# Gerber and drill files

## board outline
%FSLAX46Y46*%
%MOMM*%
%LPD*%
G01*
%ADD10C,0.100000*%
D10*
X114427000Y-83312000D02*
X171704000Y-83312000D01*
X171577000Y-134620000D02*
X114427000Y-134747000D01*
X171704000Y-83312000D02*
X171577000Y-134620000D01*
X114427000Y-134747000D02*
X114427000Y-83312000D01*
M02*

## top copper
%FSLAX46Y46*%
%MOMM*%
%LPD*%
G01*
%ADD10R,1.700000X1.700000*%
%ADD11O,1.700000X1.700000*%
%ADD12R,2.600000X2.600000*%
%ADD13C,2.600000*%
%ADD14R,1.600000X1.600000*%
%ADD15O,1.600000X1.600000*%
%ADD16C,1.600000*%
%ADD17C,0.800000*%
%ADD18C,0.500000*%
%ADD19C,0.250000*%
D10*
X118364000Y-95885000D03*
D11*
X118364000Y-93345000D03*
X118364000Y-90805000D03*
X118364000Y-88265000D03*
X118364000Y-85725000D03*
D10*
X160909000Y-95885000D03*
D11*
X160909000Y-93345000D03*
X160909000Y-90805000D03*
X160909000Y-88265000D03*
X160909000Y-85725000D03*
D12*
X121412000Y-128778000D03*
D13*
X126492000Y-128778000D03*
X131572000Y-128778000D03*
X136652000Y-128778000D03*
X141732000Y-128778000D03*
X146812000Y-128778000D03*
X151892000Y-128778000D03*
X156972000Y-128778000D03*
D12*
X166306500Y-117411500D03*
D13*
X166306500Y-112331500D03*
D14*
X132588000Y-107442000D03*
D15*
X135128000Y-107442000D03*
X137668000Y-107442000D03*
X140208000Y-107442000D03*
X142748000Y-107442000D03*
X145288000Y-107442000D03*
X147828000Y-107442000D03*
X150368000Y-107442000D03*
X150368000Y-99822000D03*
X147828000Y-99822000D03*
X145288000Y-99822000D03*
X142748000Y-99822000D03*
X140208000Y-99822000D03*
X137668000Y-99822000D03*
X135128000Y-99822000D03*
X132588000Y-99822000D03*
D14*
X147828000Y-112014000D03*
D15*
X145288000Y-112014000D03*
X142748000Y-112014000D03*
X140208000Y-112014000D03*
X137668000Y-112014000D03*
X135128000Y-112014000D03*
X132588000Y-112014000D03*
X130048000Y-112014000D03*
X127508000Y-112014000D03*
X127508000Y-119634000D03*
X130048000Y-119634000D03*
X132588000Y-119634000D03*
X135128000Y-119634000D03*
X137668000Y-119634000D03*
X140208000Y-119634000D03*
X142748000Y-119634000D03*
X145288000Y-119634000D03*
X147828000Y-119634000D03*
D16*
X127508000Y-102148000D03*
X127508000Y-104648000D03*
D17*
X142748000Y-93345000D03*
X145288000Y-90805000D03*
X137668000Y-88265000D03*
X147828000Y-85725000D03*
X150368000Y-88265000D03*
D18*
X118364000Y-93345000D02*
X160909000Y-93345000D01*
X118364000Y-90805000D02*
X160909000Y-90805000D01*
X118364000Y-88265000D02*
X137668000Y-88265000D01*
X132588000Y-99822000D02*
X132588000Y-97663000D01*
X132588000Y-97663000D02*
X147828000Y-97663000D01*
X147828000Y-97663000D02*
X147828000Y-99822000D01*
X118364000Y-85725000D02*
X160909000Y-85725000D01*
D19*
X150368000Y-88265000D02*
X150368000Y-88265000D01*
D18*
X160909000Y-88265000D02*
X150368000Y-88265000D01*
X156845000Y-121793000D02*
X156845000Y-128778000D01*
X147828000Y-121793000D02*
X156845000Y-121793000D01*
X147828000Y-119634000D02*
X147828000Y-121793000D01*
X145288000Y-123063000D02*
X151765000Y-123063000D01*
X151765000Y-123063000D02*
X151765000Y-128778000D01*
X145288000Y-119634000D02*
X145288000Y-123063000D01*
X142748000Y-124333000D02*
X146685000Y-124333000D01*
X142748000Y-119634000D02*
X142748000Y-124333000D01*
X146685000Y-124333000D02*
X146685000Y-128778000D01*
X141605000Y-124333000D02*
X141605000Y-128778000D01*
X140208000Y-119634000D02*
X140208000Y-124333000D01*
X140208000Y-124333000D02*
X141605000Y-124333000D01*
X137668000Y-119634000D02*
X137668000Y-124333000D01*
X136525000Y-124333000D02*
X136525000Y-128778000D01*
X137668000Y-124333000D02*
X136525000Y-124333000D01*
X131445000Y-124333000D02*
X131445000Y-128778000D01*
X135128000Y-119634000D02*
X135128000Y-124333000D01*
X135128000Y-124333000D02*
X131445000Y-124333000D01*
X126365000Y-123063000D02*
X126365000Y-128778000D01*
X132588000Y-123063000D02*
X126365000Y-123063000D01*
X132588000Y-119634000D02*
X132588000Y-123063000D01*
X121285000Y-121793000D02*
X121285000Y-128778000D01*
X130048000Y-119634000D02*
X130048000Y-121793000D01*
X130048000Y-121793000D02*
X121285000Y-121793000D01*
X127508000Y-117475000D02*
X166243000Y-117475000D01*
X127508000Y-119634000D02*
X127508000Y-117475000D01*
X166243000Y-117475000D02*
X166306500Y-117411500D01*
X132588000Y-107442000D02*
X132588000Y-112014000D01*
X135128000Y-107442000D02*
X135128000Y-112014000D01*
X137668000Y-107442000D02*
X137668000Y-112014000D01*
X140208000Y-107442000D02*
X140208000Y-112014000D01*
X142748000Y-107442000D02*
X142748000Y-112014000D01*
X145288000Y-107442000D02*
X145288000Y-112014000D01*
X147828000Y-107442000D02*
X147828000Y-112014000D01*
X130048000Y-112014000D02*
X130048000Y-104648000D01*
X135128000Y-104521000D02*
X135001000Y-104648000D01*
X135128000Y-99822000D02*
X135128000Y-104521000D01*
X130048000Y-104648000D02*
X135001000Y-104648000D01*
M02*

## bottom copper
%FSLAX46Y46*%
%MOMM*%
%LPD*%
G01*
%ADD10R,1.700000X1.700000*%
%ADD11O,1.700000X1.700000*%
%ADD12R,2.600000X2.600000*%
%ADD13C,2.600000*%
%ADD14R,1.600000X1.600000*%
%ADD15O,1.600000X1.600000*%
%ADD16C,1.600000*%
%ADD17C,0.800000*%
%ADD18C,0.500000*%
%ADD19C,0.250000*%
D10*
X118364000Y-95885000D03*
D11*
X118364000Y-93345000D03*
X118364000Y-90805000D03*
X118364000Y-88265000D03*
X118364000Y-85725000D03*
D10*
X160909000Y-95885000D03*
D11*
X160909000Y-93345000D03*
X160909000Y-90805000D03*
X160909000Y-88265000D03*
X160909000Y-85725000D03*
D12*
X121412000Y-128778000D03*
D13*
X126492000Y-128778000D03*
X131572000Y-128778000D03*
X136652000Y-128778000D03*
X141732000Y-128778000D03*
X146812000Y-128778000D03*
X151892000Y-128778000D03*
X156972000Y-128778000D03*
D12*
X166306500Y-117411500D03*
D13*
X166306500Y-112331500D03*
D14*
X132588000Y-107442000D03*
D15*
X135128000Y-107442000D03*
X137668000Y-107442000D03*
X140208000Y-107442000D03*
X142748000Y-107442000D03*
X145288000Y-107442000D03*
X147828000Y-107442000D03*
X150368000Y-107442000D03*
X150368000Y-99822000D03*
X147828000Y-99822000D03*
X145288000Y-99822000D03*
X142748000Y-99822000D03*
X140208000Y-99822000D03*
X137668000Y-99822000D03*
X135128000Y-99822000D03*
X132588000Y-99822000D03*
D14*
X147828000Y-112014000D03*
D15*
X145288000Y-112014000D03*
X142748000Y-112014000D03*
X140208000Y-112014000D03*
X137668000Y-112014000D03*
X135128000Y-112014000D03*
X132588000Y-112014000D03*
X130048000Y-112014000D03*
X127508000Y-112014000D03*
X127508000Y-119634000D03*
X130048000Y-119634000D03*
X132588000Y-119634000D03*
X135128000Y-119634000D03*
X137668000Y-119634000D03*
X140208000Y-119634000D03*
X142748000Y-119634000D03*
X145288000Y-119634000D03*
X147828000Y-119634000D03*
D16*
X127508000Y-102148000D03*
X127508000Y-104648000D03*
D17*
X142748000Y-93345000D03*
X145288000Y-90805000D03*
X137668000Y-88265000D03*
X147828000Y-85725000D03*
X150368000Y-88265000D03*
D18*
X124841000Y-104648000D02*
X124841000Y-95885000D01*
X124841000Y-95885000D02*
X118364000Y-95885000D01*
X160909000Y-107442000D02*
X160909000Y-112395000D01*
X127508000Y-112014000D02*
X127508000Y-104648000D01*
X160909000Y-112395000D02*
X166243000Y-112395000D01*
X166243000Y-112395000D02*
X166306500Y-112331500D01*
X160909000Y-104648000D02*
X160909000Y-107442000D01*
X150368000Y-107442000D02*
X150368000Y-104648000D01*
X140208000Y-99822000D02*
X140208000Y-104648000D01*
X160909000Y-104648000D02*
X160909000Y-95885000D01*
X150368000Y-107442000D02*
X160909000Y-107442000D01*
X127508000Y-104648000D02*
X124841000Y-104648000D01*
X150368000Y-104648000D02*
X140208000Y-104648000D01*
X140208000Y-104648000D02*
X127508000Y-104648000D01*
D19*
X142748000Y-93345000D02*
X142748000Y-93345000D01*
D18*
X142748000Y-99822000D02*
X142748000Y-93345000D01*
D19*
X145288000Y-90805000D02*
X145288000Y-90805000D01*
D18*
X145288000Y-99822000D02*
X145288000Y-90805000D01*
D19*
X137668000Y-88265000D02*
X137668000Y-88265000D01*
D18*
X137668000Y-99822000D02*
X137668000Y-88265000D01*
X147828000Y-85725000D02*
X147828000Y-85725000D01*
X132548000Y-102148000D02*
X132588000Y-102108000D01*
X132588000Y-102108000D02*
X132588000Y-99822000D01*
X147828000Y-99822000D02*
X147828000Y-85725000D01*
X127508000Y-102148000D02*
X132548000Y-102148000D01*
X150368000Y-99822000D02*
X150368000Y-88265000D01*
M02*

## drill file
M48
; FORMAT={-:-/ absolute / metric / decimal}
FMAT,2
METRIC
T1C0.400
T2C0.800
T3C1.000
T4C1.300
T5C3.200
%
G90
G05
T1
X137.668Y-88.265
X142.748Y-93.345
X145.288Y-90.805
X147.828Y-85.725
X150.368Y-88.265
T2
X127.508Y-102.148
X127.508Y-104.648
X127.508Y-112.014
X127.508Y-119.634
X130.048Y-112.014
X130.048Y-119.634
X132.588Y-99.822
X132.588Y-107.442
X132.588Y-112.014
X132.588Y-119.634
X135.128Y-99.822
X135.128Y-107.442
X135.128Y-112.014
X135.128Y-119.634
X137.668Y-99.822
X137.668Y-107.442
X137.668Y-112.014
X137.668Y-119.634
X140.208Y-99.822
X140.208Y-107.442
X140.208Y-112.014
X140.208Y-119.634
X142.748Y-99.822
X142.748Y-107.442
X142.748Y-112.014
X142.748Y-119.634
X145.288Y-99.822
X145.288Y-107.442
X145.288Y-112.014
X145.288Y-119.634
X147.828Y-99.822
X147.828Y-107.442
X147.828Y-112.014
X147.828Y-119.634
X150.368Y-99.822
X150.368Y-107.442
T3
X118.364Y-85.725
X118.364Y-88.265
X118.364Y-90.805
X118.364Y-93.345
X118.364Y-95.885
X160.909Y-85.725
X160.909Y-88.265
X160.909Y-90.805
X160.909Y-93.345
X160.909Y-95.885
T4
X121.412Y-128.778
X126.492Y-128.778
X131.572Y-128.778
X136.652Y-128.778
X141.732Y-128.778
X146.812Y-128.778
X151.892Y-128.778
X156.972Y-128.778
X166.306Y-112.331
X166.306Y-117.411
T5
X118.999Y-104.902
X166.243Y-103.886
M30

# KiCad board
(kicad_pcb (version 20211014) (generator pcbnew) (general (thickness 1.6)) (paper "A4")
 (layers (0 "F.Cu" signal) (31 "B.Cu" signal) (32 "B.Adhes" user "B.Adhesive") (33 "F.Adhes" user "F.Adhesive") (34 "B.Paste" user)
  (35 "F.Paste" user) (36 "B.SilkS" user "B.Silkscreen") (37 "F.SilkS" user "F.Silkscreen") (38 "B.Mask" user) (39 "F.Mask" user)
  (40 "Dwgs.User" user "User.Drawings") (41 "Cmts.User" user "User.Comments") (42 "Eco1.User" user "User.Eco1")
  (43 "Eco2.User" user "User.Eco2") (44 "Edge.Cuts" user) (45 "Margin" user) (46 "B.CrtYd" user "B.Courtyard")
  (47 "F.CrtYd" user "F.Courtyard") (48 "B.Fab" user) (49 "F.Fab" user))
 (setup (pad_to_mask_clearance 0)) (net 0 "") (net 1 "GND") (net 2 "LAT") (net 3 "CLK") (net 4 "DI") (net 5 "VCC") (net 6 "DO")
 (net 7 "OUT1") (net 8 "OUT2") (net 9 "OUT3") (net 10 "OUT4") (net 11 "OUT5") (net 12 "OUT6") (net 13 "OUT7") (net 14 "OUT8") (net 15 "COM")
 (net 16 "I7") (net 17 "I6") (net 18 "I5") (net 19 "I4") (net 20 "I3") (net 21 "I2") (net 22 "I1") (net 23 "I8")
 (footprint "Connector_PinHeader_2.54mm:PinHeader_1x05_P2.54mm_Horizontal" (layer "F.Cu") (at 118.364 95.885 180)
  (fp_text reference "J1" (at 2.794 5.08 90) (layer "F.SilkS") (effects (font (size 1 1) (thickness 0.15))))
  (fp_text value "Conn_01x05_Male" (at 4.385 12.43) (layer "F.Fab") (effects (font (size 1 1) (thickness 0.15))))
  (pad "1" thru_hole rect locked (at 0 0 180) (size 1.7 1.7) (drill 1) (layers *.Cu *.Mask) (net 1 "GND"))
  (pad "2" thru_hole oval locked (at 0 2.54 180) (size 1.7 1.7) (drill 1) (layers *.Cu *.Mask) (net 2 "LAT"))
  (pad "3" thru_hole oval locked (at 0 5.08 180) (size 1.7 1.7) (drill 1) (layers *.Cu *.Mask) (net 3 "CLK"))
  (pad "4" thru_hole oval locked (at 0 7.62 180) (size 1.7 1.7) (drill 1) (layers *.Cu *.Mask) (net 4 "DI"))
  (pad "5" thru_hole oval locked (at 0 10.16 180) (size 1.7 1.7) (drill 1) (layers *.Cu *.Mask) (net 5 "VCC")))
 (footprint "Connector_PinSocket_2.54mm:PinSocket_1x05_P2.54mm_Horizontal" (layer "F.Cu") (at 160.909 95.885 180)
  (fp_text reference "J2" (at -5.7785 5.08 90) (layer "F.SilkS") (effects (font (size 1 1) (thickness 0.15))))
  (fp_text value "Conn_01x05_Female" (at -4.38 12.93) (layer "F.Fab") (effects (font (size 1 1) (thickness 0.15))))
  (pad "1" thru_hole rect locked (at 0 0 180) (size 1.7 1.7) (drill 1) (layers *.Cu *.Mask) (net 1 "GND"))
  (pad "2" thru_hole oval locked (at 0 2.54 180) (size 1.7 1.7) (drill 1) (layers *.Cu *.Mask) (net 2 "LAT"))
  (pad "3" thru_hole oval locked (at 0 5.08 180) (size 1.7 1.7) (drill 1) (layers *.Cu *.Mask) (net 3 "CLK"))
  (pad "4" thru_hole oval locked (at 0 7.62 180) (size 1.7 1.7) (drill 1) (layers *.Cu *.Mask) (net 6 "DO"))
  (pad "5" thru_hole oval locked (at 0 10.16 180) (size 1.7 1.7) (drill 1) (layers *.Cu *.Mask) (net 5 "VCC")))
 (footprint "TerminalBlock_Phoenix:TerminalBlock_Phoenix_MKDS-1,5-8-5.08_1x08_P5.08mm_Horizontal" (layer "F.Cu") (at 121.412 128.778)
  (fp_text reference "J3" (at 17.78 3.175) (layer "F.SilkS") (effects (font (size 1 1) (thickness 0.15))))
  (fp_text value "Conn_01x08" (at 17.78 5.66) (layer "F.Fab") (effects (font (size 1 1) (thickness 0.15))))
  (pad "1" thru_hole rect locked (at 0 0) (size 2.6 2.6) (drill 1.3) (layers *.Cu *.Mask) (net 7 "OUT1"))
  (pad "2" thru_hole circle locked (at 5.08 0) (size 2.6 2.6) (drill 1.3) (layers *.Cu *.Mask) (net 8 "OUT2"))
  (pad "3" thru_hole circle locked (at 10.16 0) (size 2.6 2.6) (drill 1.3) (layers *.Cu *.Mask) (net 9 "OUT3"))
  (pad "4" thru_hole circle locked (at 15.24 0) (size 2.6 2.6) (drill 1.3) (layers *.Cu *.Mask) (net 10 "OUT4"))
  (pad "5" thru_hole circle locked (at 20.32 0) (size 2.6 2.6) (drill 1.3) (layers *.Cu *.Mask) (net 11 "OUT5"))
  (pad "6" thru_hole circle locked (at 25.4 0) (size 2.6 2.6) (drill 1.3) (layers *.Cu *.Mask) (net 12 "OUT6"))
  (pad "7" thru_hole circle locked (at 30.48 0) (size 2.6 2.6) (drill 1.3) (layers *.Cu *.Mask) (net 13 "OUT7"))
  (pad "8" thru_hole circle locked (at 35.56 0) (size 2.6 2.6) (drill 1.3) (layers *.Cu *.Mask) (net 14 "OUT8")))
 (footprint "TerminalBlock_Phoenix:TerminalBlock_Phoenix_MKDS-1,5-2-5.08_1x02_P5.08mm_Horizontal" (layer "F.Cu") (at 166.3065 117.4115 90)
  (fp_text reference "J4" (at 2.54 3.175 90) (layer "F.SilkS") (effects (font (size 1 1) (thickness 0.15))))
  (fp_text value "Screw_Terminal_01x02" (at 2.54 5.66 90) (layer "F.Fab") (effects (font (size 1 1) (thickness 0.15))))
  (pad "1" thru_hole rect locked (at 0 0 90) (size 2.6 2.6) (drill 1.3) (layers *.Cu *.Mask) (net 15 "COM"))
  (pad "2" thru_hole circle locked (at 5.08 0 90) (size 2.6 2.6) (drill 1.3) (layers *.Cu *.Mask) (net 1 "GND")))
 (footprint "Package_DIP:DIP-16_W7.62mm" (layer "F.Cu") (at 132.588 107.442 90)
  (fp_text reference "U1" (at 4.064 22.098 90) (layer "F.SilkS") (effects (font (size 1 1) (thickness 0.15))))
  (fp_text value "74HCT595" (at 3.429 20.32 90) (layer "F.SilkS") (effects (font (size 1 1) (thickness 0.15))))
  (pad "1" thru_hole rect locked (at 0 0 90) (size 1.6 1.6) (drill 0.8) (layers *.Cu *.Mask) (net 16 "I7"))
  (pad "2" thru_hole oval locked (at 0 2.54 90) (size 1.6 1.6) (drill 0.8) (layers *.Cu *.Mask) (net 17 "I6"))
  (pad "3" thru_hole oval locked (at 0 5.08 90) (size 1.6 1.6) (drill 0.8) (layers *.Cu *.Mask) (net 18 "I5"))
  (pad "4" thru_hole oval locked (at 0 7.62 90) (size 1.6 1.6) (drill 0.8) (layers *.Cu *.Mask) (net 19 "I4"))
  (pad "5" thru_hole oval locked (at 0 10.16 90) (size 1.6 1.6) (drill 0.8) (layers *.Cu *.Mask) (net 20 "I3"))
  (pad "6" thru_hole oval locked (at 0 12.7 90) (size 1.6 1.6) (drill 0.8) (layers *.Cu *.Mask) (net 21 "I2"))
  (pad "7" thru_hole oval locked (at 0 15.24 90) (size 1.6 1.6) (drill 0.8) (layers *.Cu *.Mask) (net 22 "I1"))
  (pad "8" thru_hole oval locked (at 0 17.78 90) (size 1.6 1.6) (drill 0.8) (layers *.Cu *.Mask) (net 1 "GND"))
  (pad "9" thru_hole oval locked (at 7.62 17.78 90) (size 1.6 1.6) (drill 0.8) (layers *.Cu *.Mask) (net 6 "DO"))
  (pad "10" thru_hole oval locked (at 7.62 15.24 90) (size 1.6 1.6) (drill 0.8) (layers *.Cu *.Mask) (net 5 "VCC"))
  (pad "11" thru_hole oval locked (at 7.62 12.7 90) (size 1.6 1.6) (drill 0.8) (layers *.Cu *.Mask) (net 3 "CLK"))
  (pad "12" thru_hole oval locked (at 7.62 10.16 90) (size 1.6 1.6) (drill 0.8) (layers *.Cu *.Mask) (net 2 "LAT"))
  (pad "13" thru_hole oval locked (at 7.62 7.62 90) (size 1.6 1.6) (drill 0.8) (layers *.Cu *.Mask) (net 1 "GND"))
  (pad "14" thru_hole oval locked (at 7.62 5.08 90) (size 1.6 1.6) (drill 0.8) (layers *.Cu *.Mask) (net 4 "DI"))
  (pad "15" thru_hole oval locked (at 7.62 2.54 90) (size 1.6 1.6) (drill 0.8) (layers *.Cu *.Mask) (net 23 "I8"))
  (pad "16" thru_hole oval locked (at 7.62 0 90) (size 1.6 1.6) (drill 0.8) (layers *.Cu *.Mask) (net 5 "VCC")))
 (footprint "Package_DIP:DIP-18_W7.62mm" (layer "F.Cu") (at 147.828 112.014 -90)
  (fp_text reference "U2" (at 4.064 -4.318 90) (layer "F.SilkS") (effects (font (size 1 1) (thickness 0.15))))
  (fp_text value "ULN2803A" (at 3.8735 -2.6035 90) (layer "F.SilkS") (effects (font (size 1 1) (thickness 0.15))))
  (pad "1" thru_hole rect locked (at 0 0 270) (size 1.6 1.6) (drill 0.8) (layers *.Cu *.Mask) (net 22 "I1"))
  (pad "2" thru_hole oval locked (at 0 2.54 270) (size 1.6 1.6) (drill 0.8) (layers *.Cu *.Mask) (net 21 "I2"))
  (pad "3" thru_hole oval locked (at 0 5.08 270) (size 1.6 1.6) (drill 0.8) (layers *.Cu *.Mask) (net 20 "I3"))
  (pad "4" thru_hole oval locked (at 0 7.62 270) (size 1.6 1.6) (drill 0.8) (layers *.Cu *.Mask) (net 19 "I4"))
  (pad "5" thru_hole oval locked (at 0 10.16 270) (size 1.6 1.6) (drill 0.8) (layers *.Cu *.Mask) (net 18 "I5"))
  (pad "6" thru_hole oval locked (at 0 12.7 270) (size 1.6 1.6) (drill 0.8) (layers *.Cu *.Mask) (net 17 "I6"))
  (pad "7" thru_hole oval locked (at 0 15.24 270) (size 1.6 1.6) (drill 0.8) (layers *.Cu *.Mask) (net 16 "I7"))
  (pad "8" thru_hole oval locked (at 0 17.78 270) (size 1.6 1.6) (drill 0.8) (layers *.Cu *.Mask) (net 23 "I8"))
  (pad "9" thru_hole oval locked (at 0 20.32 270) (size 1.6 1.6) (drill 0.8) (layers *.Cu *.Mask) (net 1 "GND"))
  (pad "10" thru_hole oval locked (at 7.62 20.32 270) (size 1.6 1.6) (drill 0.8) (layers *.Cu *.Mask) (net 15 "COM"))
  (pad "11" thru_hole oval locked (at 7.62 17.78 270) (size 1.6 1.6) (drill 0.8) (layers *.Cu *.Mask) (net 7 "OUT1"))
  (pad "12" thru_hole oval locked (at 7.62 15.24 270) (size 1.6 1.6) (drill 0.8) (layers *.Cu *.Mask) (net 8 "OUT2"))
  (pad "13" thru_hole oval locked (at 7.62 12.7 270) (size 1.6 1.6) (drill 0.8) (layers *.Cu *.Mask) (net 9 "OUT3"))
  (pad "14" thru_hole oval locked (at 7.62 10.16 270) (size 1.6 1.6) (drill 0.8) (layers *.Cu *.Mask) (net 10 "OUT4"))
  (pad "15" thru_hole oval locked (at 7.62 7.62 270) (size 1.6 1.6) (drill 0.8) (layers *.Cu *.Mask) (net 11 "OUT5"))
  (pad "16" thru_hole oval locked (at 7.62 5.08 270) (size 1.6 1.6) (drill 0.8) (layers *.Cu *.Mask) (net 12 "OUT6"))
  (pad "17" thru_hole oval locked (at 7.62 2.54 270) (size 1.6 1.6) (drill 0.8) (layers *.Cu *.Mask) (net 13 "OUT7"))
  (pad "18" thru_hole oval locked (at 7.62 0 270) (size 1.6 1.6) (drill 0.8) (layers *.Cu *.Mask) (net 14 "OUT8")))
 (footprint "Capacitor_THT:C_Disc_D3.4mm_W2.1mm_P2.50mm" (layer "F.Cu") (at 127.508 102.148 -90)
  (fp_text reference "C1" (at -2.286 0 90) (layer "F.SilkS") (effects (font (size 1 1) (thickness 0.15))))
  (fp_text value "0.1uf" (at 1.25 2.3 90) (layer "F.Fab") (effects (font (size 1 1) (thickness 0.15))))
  (pad "1" thru_hole circle locked (at 0 0 270) (size 1.6 1.6) (drill 0.8) (layers *.Cu *.Mask) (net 5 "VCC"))
  (pad "2" thru_hole circle locked (at 2.5 0 270) (size 1.6 1.6) (drill 0.8) (layers *.Cu *.Mask) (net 1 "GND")))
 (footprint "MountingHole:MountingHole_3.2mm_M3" (layer "F.Cu") (at 118.999 104.902)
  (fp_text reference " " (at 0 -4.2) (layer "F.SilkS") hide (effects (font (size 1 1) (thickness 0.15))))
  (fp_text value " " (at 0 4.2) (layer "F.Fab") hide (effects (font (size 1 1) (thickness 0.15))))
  (pad "" np_thru_hole circle locked (at 0 0) (size 3.2 3.2) (drill 3.2) (layers *.Cu *.Mask)))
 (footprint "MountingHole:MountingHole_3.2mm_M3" (layer "F.Cu") (at 166.243 103.886)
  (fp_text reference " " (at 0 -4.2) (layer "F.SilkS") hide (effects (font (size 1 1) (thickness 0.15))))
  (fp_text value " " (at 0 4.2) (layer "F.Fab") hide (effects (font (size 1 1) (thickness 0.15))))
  (pad "" np_thru_hole circle locked (at 0 0) (size 3.2 3.2) (drill 3.2) (layers *.Cu *.Mask)))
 (gr_line (start 114.427 83.312) (end 171.704 83.312) (layer "Edge.Cuts") (width 0.1))
 (gr_line (start 171.577 134.62) (end 114.427 134.747) (layer "Edge.Cuts") (width 0.1))
 (gr_line (start 171.704 83.312) (end 171.577 134.62) (layer "Edge.Cuts") (width 0.1))
 (gr_line (start 114.427 134.747) (end 114.427 83.312) (layer "Edge.Cuts") (width 0.1))
 (segment (start 124.841 104.648) (end 124.841 95.885) (width 0.5) (layer "B.Cu") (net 1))
 (segment (start 124.841 95.885) (end 118.364 95.885) (width 0.5) (layer "B.Cu") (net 1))
 (segment (start 160.909 107.442) (end 160.909 112.395) (width 0.5) (layer "B.Cu") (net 1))
 (segment (start 127.508 112.014) (end 127.508 104.648) (width 0.5) (layer "B.Cu") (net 1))
 (segment (start 160.909 112.395) (end 166.243 112.395) (width 0.5) (layer "B.Cu") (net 1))
 (segment (start 166.243 112.395) (end 166.3065 112.3315) (width 0.5) (layer "B.Cu") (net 1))
 (segment (start 160.909 104.648) (end 160.909 107.442) (width 0.5) (layer "B.Cu") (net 1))
 (segment (start 150.368 107.442) (end 150.368 104.648) (width 0.5) (layer "B.Cu") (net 1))
 (segment (start 140.208 99.822) (end 140.208 104.648) (width 0.5) (layer "B.Cu") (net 1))
 (segment (start 160.909 104.648) (end 160.909 95.885) (width 0.5) (layer "B.Cu") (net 1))
 (segment (start 150.368 107.442) (end 160.909 107.442) (width 0.5) (layer "B.Cu") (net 1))
 (segment (start 127.508 104.648) (end 124.841 104.648) (width 0.5) (layer "B.Cu") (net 1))
 (segment (start 150.368 104.648) (end 140.208 104.648) (width 0.5) (layer "B.Cu") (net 1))
 (segment (start 140.208 104.648) (end 127.508 104.648) (width 0.5) (layer "B.Cu") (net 1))
 (segment (start 118.364 93.345) (end 160.909 93.345) (width 0.5) (layer "F.Cu") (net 2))
 (via (at 142.748 93.345) (size 0.8) (drill 0.4) (layers "F.Cu" "B.Cu") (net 2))
 (segment (start 142.748 93.345) (end 142.748 93.345) (width 0.25) (layer "B.Cu") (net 2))
 (segment (start 142.748 99.822) (end 142.748 93.345) (width 0.5) (layer "B.Cu") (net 2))
 (segment (start 118.364 90.805) (end 160.909 90.805) (width 0.5) (layer "F.Cu") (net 3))
 (via (at 145.288 90.805) (size 0.8) (drill 0.4) (layers "F.Cu" "B.Cu") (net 3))
 (segment (start 145.288 90.805) (end 145.288 90.805) (width 0.25) (layer "B.Cu") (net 3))
 (segment (start 145.288 99.822) (end 145.288 90.805) (width 0.5) (layer "B.Cu") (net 3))
 (segment (start 118.364 88.265) (end 137.668 88.265) (width 0.5) (layer "F.Cu") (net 4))
 (via (at 137.668 88.265) (size 0.8) (drill 0.4) (layers "F.Cu" "B.Cu") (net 4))
 (segment (start 137.668 88.265) (end 137.668 88.265) (width 0.25) (layer "B.Cu") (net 4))
 (segment (start 137.668 99.822) (end 137.668 88.265) (width 0.5) (layer "B.Cu") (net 4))
 (segment (start 132.588 99.822) (end 132.588 97.663) (width 0.5) (layer "F.Cu") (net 5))
 (segment (start 132.588 97.663) (end 147.828 97.663) (width 0.5) (layer "F.Cu") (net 5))
 (segment (start 147.828 97.663) (end 147.828 99.822) (width 0.5) (layer "F.Cu") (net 5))
 (segment (start 118.364 85.725) (end 160.909 85.725) (width 0.5) (layer "F.Cu") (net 5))
 (via (at 147.828 85.725) (size 0.8) (drill 0.4) (layers "F.Cu" "B.Cu") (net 5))
 (segment (start 147.828 85.725) (end 147.828 85.725) (width 0.5) (layer "B.Cu") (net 5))
 (segment (start 132.548 102.148) (end 132.588 102.108) (width 0.5) (layer "B.Cu") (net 5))
 (segment (start 132.588 102.108) (end 132.588 99.822) (width 0.5) (layer "B.Cu") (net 5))
 (segment (start 147.828 99.822) (end 147.828 85.725) (width 0.5) (layer "B.Cu") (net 5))
 (segment (start 127.508 102.148) (end 132.548 102.148) (width 0.5) (layer "B.Cu") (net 5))
 (segment (start 150.368 88.265) (end 150.368 88.265) (width 0.25) (layer "F.Cu") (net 6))
 (segment (start 160.909 88.265) (end 150.368 88.265) (width 0.5) (layer "F.Cu") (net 6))
 (via (at 150.368 88.265) (size 0.8) (drill 0.4) (layers "F.Cu" "B.Cu") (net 6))
 (segment (start 150.368 99.822) (end 150.368 88.265) (width 0.5) (layer "B.Cu") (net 6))
 (segment (start 156.845 121.793) (end 156.845 128.778) (width 0.5) (layer "F.Cu") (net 14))
 (segment (start 147.828 121.793) (end 156.845 121.793) (width 0.5) (layer "F.Cu") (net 14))
 (segment (start 147.828 119.634) (end 147.828 121.793) (width 0.5) (layer "F.Cu") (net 14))
 (segment (start 145.288 123.063) (end 151.765 123.063) (width 0.5) (layer "F.Cu") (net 13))
 (segment (start 151.765 123.063) (end 151.765 128.778) (width 0.5) (layer "F.Cu") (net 13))
 (segment (start 145.288 119.634) (end 145.288 123.063) (width 0.5) (layer "F.Cu") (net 13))
 (segment (start 142.748 124.333) (end 146.685 124.333) (width 0.5) (layer "F.Cu") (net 12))
 (segment (start 142.748 119.634) (end 142.748 124.333) (width 0.5) (layer "F.Cu") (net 12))
 (segment (start 146.685 124.333) (end 146.685 128.778) (width 0.5) (layer "F.Cu") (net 12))
 (segment (start 141.605 124.333) (end 141.605 128.778) (width 0.5) (layer "F.Cu") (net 11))
 (segment (start 140.208 119.634) (end 140.208 124.333) (width 0.5) (layer "F.Cu") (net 11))
 (segment (start 140.208 124.333) (end 141.605 124.333) (width 0.5) (layer "F.Cu") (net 11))
 (segment (start 137.668 119.634) (end 137.668 124.333) (width 0.5) (layer "F.Cu") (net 10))
 (segment (start 136.525 124.333) (end 136.525 128.778) (width 0.5) (layer "F.Cu") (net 10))
 (segment (start 137.668 124.333) (end 136.525 124.333) (width 0.5) (layer "F.Cu") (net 10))
 (segment (start 131.445 124.333) (end 131.445 128.778) (width 0.5) (layer "F.Cu") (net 9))
 (segment (start 135.128 119.634) (end 135.128 124.333) (width 0.5) (layer "F.Cu") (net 9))
 (segment (start 135.128 124.333) (end 131.445 124.333) (width 0.5) (layer "F.Cu") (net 9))
 (segment (start 126.365 123.063) (end 126.365 128.778) (width 0.5) (layer "F.Cu") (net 8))
 (segment (start 132.588 123.063) (end 126.365 123.063) (width 0.5) (layer "F.Cu") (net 8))
 (segment (start 132.588 119.634) (end 132.588 123.063) (width 0.5) (layer "F.Cu") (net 8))
 (segment (start 121.285 121.793) (end 121.285 128.778) (width 0.5) (layer "F.Cu") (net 7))
 (segment (start 130.048 119.634) (end 130.048 121.793) (width 0.5) (layer "F.Cu") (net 7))
 (segment (start 130.048 121.793) (end 121.285 121.793) (width 0.5) (layer "F.Cu") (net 7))
 (segment (start 127.508 117.475) (end 166.243 117.475) (width 0.5) (layer "F.Cu") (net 15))
 (segment (start 127.508 119.634) (end 127.508 117.475) (width 0.5) (layer "F.Cu") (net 15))
 (segment (start 166.243 117.475) (end 166.3065 117.4115) (width 0.5) (layer "F.Cu") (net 15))
 (segment (start 132.588 107.442) (end 132.588 112.014) (width 0.5) (layer "F.Cu") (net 16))
 (segment (start 135.128 107.442) (end 135.128 112.014) (width 0.5) (layer "F.Cu") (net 17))
 (segment (start 137.668 107.442) (end 137.668 112.014) (width 0.5) (layer "F.Cu") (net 18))
 (segment (start 140.208 107.442) (end 140.208 112.014) (width 0.5) (layer "F.Cu") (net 19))
 (segment (start 142.748 107.442) (end 142.748 112.014) (width 0.5) (layer "F.Cu") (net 20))
 (segment (start 145.288 107.442) (end 145.288 112.014) (width 0.5) (layer "F.Cu") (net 21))
 (segment (start 147.828 107.442) (end 147.828 112.014) (width 0.5) (layer "F.Cu") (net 22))
 (segment (start 130.048 112.014) (end 130.048 104.648) (width 0.5) (layer "F.Cu") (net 23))
 (segment (start 135.128 104.521) (end 135.001 104.648) (width 0.5) (layer "F.Cu") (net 23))
 (segment (start 135.128 99.822) (end 135.128 104.521) (width 0.5) (layer "F.Cu") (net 23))
 (segment (start 130.048 104.648) (end 135.001 104.648) (width 0.5) (layer "F.Cu") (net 23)))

